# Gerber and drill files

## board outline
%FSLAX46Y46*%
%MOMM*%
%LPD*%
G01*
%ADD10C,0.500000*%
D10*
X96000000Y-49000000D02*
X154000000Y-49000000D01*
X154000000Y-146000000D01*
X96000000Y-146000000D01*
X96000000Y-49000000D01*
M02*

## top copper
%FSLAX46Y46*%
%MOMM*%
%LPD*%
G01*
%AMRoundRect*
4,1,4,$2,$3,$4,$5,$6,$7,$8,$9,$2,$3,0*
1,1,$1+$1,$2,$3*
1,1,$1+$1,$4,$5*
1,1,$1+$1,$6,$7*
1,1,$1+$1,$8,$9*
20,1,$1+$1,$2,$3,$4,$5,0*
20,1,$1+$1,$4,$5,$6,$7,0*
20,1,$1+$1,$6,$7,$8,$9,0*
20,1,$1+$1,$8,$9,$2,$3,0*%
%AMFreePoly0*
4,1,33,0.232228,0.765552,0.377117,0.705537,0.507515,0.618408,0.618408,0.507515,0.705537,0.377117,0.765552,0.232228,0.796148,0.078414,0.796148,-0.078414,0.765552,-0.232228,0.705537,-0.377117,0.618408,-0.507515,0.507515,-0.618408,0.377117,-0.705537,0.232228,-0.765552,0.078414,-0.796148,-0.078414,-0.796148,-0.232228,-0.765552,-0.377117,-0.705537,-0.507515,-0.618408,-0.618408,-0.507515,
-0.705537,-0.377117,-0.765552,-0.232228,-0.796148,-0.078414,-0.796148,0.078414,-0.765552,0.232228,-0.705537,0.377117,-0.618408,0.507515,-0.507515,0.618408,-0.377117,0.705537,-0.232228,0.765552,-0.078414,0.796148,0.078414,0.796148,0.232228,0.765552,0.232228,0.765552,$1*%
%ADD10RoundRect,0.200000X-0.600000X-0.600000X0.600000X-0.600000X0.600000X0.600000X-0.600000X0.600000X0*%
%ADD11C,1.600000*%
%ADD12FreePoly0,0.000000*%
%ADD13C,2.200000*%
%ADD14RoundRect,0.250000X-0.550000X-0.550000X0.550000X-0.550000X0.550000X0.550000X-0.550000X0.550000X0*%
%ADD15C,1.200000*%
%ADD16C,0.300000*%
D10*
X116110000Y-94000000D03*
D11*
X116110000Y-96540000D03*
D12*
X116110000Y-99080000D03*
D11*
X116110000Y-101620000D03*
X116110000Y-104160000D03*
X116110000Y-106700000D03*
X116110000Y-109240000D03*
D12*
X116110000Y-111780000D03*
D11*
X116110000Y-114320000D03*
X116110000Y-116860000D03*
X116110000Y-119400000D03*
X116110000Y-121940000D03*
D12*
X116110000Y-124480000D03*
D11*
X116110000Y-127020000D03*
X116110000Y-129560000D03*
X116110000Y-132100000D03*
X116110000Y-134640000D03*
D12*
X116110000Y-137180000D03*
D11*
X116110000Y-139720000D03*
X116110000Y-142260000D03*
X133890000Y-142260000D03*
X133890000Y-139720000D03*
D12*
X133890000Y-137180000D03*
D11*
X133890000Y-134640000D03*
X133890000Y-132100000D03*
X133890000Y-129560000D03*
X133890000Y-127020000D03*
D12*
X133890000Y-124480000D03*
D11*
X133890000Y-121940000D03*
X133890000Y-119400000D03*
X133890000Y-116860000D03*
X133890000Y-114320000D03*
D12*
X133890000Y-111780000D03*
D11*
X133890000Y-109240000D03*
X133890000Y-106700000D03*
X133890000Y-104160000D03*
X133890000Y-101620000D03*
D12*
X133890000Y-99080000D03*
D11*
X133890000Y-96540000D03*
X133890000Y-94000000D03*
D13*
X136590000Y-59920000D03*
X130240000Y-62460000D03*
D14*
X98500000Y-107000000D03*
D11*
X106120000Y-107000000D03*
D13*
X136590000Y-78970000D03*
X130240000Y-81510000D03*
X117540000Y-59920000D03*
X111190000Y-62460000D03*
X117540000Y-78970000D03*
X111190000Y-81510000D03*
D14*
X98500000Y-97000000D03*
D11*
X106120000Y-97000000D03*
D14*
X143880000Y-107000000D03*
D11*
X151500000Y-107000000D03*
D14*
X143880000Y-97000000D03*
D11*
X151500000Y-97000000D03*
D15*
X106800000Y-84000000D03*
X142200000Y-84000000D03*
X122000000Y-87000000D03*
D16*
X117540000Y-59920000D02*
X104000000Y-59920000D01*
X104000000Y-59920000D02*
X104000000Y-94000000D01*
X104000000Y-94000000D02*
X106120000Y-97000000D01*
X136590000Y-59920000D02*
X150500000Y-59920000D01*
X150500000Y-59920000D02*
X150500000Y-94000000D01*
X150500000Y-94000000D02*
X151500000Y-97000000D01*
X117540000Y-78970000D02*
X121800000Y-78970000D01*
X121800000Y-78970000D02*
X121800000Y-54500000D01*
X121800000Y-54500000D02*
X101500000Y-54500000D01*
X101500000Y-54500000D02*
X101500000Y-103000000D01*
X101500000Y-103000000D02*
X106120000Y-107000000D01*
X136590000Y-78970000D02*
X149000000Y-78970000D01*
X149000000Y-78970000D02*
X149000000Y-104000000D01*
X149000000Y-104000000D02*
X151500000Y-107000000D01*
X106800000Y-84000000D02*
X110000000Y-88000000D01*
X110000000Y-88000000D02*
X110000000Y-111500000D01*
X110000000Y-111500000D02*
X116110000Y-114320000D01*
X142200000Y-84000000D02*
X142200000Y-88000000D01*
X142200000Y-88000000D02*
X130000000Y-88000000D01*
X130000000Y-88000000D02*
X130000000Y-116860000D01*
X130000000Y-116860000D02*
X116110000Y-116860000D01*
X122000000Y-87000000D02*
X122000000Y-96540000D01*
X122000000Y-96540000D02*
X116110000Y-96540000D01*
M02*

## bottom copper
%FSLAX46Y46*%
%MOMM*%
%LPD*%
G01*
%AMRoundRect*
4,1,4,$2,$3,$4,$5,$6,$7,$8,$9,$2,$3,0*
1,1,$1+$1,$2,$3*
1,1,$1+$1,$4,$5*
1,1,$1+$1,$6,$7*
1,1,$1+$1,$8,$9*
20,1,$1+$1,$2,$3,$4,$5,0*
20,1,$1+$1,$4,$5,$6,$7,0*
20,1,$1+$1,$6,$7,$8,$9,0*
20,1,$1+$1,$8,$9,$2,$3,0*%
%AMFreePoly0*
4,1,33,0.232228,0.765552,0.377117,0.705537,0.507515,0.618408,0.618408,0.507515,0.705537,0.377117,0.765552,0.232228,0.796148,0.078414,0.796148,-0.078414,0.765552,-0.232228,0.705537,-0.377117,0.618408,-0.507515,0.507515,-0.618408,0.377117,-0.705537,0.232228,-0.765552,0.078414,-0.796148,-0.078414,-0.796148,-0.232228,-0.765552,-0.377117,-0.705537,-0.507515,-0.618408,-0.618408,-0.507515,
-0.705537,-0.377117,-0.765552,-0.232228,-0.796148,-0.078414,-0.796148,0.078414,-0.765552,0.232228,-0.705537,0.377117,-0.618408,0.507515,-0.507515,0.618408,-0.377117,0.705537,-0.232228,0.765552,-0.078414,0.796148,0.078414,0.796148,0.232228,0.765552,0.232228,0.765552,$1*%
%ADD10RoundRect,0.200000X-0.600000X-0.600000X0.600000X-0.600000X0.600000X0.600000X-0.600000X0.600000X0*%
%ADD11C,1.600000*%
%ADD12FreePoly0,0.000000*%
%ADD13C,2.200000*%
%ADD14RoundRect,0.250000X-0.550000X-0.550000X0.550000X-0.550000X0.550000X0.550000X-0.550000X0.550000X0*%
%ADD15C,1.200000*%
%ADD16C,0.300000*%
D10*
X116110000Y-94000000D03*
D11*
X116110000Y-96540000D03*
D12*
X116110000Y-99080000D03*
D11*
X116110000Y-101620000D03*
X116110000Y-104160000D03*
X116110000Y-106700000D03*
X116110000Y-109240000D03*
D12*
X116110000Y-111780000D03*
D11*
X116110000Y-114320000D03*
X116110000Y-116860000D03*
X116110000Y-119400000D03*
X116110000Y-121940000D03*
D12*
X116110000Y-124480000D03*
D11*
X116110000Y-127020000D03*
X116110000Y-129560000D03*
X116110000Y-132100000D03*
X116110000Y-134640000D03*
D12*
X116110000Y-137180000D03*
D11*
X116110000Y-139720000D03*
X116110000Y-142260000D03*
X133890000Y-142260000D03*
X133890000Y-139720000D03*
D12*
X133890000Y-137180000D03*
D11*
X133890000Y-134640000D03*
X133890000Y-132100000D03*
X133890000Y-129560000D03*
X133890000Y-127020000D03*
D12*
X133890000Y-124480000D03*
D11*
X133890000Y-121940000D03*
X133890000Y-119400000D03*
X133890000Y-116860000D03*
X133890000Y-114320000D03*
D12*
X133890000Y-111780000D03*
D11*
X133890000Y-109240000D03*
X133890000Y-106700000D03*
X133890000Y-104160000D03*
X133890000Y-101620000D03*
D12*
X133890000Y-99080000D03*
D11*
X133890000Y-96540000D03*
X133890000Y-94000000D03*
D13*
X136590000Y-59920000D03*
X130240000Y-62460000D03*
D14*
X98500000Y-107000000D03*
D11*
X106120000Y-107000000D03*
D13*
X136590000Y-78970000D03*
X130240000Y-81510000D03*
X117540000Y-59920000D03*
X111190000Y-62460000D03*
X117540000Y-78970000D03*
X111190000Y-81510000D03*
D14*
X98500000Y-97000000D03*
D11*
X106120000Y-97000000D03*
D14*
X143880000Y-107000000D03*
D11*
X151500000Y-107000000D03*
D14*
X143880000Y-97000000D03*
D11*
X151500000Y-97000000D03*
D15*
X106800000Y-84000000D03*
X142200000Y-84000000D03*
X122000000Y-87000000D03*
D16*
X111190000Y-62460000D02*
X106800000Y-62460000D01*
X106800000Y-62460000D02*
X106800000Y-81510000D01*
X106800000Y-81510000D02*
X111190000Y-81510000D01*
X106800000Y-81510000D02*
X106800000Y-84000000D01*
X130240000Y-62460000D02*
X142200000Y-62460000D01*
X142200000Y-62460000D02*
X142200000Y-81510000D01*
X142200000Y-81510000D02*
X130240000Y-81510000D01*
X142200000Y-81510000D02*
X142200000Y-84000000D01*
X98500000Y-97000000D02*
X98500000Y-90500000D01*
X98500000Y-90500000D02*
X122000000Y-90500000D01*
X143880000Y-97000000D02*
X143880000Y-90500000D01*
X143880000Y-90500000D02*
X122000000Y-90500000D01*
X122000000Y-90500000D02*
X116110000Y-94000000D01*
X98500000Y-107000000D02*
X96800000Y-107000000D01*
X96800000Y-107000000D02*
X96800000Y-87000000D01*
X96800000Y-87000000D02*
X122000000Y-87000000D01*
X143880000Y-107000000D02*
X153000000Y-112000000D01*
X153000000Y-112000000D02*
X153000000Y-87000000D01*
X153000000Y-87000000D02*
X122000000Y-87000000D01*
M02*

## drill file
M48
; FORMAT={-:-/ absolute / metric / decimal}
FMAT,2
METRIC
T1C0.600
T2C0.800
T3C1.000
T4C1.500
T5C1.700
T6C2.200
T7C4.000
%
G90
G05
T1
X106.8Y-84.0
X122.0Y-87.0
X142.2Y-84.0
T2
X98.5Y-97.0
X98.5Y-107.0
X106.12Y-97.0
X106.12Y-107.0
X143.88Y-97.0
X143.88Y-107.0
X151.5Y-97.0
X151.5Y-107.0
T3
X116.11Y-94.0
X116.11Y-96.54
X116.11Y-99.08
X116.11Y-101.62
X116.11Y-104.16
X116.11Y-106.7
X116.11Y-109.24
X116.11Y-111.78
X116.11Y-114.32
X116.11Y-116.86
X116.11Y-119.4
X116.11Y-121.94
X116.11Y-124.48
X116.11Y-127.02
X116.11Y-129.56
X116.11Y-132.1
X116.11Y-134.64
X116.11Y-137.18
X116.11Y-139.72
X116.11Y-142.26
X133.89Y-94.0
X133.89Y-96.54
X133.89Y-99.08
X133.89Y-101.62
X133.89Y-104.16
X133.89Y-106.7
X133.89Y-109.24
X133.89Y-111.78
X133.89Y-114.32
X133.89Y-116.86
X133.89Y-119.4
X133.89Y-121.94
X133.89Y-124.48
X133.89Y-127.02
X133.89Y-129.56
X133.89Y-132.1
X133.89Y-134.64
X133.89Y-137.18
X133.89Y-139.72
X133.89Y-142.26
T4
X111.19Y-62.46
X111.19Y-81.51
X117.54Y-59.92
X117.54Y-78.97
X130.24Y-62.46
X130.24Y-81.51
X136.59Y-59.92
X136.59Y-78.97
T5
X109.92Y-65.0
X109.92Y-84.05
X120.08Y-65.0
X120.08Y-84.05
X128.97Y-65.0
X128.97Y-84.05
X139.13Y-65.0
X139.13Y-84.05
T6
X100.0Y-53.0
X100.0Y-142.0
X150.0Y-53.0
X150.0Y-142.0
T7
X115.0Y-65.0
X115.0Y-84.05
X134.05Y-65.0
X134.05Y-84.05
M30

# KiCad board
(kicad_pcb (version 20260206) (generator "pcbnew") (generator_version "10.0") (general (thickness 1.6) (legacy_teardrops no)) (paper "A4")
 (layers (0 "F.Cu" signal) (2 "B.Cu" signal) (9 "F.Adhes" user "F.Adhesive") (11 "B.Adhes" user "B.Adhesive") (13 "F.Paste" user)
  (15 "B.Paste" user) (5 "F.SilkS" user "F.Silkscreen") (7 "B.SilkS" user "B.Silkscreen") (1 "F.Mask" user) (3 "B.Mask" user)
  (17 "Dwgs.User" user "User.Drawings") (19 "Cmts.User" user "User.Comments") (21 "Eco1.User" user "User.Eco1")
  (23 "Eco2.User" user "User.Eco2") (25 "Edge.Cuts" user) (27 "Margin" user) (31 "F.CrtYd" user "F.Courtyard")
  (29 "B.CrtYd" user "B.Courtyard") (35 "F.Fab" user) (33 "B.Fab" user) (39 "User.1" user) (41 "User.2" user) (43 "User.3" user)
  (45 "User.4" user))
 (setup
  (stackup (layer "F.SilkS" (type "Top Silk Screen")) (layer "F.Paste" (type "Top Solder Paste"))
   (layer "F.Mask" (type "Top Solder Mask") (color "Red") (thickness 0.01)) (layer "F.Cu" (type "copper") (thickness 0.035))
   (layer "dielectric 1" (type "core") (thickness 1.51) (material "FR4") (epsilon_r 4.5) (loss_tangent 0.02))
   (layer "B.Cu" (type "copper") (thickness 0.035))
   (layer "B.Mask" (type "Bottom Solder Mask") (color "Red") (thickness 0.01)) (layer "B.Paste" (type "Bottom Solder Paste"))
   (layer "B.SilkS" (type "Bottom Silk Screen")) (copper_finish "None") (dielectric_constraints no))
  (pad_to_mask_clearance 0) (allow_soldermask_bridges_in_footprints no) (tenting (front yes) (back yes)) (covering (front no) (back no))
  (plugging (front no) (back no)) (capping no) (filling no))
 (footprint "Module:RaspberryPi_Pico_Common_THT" (layer "F.Cu") (at 116.11 94)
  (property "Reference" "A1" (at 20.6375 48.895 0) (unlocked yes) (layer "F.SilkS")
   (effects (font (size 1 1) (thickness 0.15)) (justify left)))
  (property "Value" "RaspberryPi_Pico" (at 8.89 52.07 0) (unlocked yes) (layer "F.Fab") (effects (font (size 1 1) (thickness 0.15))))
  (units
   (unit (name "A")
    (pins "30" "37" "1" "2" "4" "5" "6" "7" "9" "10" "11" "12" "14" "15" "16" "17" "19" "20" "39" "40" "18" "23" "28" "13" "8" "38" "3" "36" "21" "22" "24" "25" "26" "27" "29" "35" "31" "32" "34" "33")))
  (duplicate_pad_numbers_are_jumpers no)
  (pad "1" thru_hole roundrect (at 0 0) (size 1.6 1.6) (drill 1) (layers "*.Cu" "*.Mask") (remove_unused_layers no) (roundrect_rratio 0.125)
   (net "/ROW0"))
  (pad "2" thru_hole circle (at 0 2.54) (size 1.6 1.6) (drill 1) (layers "*.Cu" "*.Mask") (remove_unused_layers no) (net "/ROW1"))
  (pad "3" thru_hole custom (at 0 5.08) (size 1.6 1.6) (drill 1) (layers "*.Cu" "*.Mask") (remove_unused_layers no)
   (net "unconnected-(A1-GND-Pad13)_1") (options (clearance outline) (anchor circle)) (primitives))
  (pad "4" thru_hole circle (at 0 7.62) (size 1.6 1.6) (drill 1) (layers "*.Cu" "*.Mask") (remove_unused_layers no)
   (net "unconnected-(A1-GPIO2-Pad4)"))
  (pad "5" thru_hole circle (at 0 10.16) (size 1.6 1.6) (drill 1) (layers "*.Cu" "*.Mask") (remove_unused_layers no)
   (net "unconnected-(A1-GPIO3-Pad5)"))
  (pad "6" thru_hole circle (at 0 12.7) (size 1.6 1.6) (drill 1) (layers "*.Cu" "*.Mask") (remove_unused_layers no)
   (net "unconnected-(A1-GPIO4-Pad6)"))
  (pad "7" thru_hole circle (at 0 15.24) (size 1.6 1.6) (drill 1) (layers "*.Cu" "*.Mask") (remove_unused_layers no)
   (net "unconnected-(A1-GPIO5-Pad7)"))
  (pad "8" thru_hole custom (at 0 17.78) (size 1.6 1.6) (drill 1) (layers "*.Cu" "*.Mask") (remove_unused_layers no)
   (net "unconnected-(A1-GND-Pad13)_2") (options (clearance outline) (anchor circle)) (primitives))
  (pad "9" thru_hole circle (at 0 20.32) (size 1.6 1.6) (drill 1) (layers "*.Cu" "*.Mask") (remove_unused_layers no) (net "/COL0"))
  (pad "10" thru_hole circle (at 0 22.86) (size 1.6 1.6) (drill 1) (layers "*.Cu" "*.Mask") (remove_unused_layers no) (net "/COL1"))
  (pad "11" thru_hole circle (at 0 25.4) (size 1.6 1.6) (drill 1) (layers "*.Cu" "*.Mask") (remove_unused_layers no)
   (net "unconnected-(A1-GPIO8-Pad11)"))
  (pad "12" thru_hole circle (at 0 27.94) (size 1.6 1.6) (drill 1) (layers "*.Cu" "*.Mask") (remove_unused_layers no)
   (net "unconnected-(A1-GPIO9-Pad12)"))
  (pad "13" thru_hole custom (at 0 30.48) (size 1.6 1.6) (drill 1) (layers "*.Cu" "*.Mask") (remove_unused_layers no)
   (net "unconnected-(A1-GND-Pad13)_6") (options (clearance outline) (anchor circle)) (primitives))
  (pad "14" thru_hole circle (at 0 33.02) (size 1.6 1.6) (drill 1) (layers "*.Cu" "*.Mask") (remove_unused_layers no)
   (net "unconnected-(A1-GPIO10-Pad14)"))
  (pad "15" thru_hole circle (at 0 35.56) (size 1.6 1.6) (drill 1) (layers "*.Cu" "*.Mask") (remove_unused_layers no)
   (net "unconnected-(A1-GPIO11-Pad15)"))
  (pad "16" thru_hole circle (at 0 38.1) (size 1.6 1.6) (drill 1) (layers "*.Cu" "*.Mask") (remove_unused_layers no)
   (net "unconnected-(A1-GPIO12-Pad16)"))
  (pad "17" thru_hole circle (at 0 40.64) (size 1.6 1.6) (drill 1) (layers "*.Cu" "*.Mask") (remove_unused_layers no)
   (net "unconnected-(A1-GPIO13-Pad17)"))
  (pad "18" thru_hole custom (at 0 43.18) (size 1.6 1.6) (drill 1) (layers "*.Cu" "*.Mask") (remove_unused_layers no)
   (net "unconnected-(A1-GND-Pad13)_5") (options (clearance outline) (anchor circle)) (primitives))
  (pad "19" thru_hole circle (at 0 45.72) (size 1.6 1.6) (drill 1) (layers "*.Cu" "*.Mask") (remove_unused_layers no)
   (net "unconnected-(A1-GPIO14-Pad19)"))
  (pad "20" thru_hole circle (at 0 48.26) (size 1.6 1.6) (drill 1) (layers "*.Cu" "*.Mask") (remove_unused_layers no)
   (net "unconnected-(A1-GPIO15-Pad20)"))
  (pad "21" thru_hole circle (at 17.78 48.26) (size 1.6 1.6) (drill 1) (layers "*.Cu" "*.Mask") (remove_unused_layers no)
   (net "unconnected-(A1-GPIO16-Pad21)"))
  (pad "22" thru_hole circle (at 17.78 45.72) (size 1.6 1.6) (drill 1) (layers "*.Cu" "*.Mask") (remove_unused_layers no)
   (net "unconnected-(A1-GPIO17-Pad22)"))
  (pad "23" thru_hole custom (at 17.78 43.18) (size 1.6 1.6) (drill 1) (layers "*.Cu" "*.Mask") (remove_unused_layers no)
   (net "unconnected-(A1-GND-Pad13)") (options (clearance outline) (anchor circle)) (primitives))
  (pad "24" thru_hole circle (at 17.78 40.64) (size 1.6 1.6) (drill 1) (layers "*.Cu" "*.Mask") (remove_unused_layers no)
   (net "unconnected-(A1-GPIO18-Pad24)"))
  (pad "25" thru_hole circle (at 17.78 38.1) (size 1.6 1.6) (drill 1) (layers "*.Cu" "*.Mask") (remove_unused_layers no)
   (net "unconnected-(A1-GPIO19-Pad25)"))
  (pad "26" thru_hole circle (at 17.78 35.56) (size 1.6 1.6) (drill 1) (layers "*.Cu" "*.Mask") (remove_unused_layers no)
   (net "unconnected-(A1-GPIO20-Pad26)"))
  (pad "27" thru_hole circle (at 17.78 33.02) (size 1.6 1.6) (drill 1) (layers "*.Cu" "*.Mask") (remove_unused_layers no)
   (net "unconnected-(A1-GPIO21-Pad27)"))
  (pad "28" thru_hole custom (at 17.78 30.48) (size 1.6 1.6) (drill 1) (layers "*.Cu" "*.Mask") (remove_unused_layers no)
   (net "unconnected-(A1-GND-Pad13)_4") (options (clearance outline) (anchor circle)) (primitives))
  (pad "29" thru_hole circle (at 17.78 27.94) (size 1.6 1.6) (drill 1) (layers "*.Cu" "*.Mask") (remove_unused_layers no)
   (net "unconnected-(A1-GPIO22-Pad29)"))
  (pad "30" thru_hole circle (at 17.78 25.4) (size 1.6 1.6) (drill 1) (layers "*.Cu" "*.Mask") (remove_unused_layers no)
   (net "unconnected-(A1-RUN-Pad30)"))
  (pad "31" thru_hole circle (at 17.78 22.86) (size 1.6 1.6) (drill 1) (layers "*.Cu" "*.Mask") (remove_unused_layers no)
   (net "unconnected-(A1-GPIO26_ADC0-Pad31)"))
  (pad "32" thru_hole circle (at 17.78 20.32) (size 1.6 1.6) (drill 1) (layers "*.Cu" "*.Mask") (remove_unused_layers no)
   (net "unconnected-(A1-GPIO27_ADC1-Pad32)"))
  (pad "33" thru_hole custom (at 17.78 17.78) (size 1.6 1.6) (drill 1) (layers "*.Cu" "*.Mask") (remove_unused_layers no)
   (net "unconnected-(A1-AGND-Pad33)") (options (clearance outline) (anchor circle)) (primitives))
  (pad "34" thru_hole circle (at 17.78 15.24) (size 1.6 1.6) (drill 1) (layers "*.Cu" "*.Mask") (remove_unused_layers no)
   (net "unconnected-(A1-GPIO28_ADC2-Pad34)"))
  (pad "35" thru_hole circle (at 17.78 12.7) (size 1.6 1.6) (drill 1) (layers "*.Cu" "*.Mask") (remove_unused_layers no)
   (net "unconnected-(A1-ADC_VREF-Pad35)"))
  (pad "36" thru_hole circle (at 17.78 10.16) (size 1.6 1.6) (drill 1) (layers "*.Cu" "*.Mask") (remove_unused_layers no)
   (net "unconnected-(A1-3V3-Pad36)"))
  (pad "37" thru_hole circle (at 17.78 7.62) (size 1.6 1.6) (drill 1) (layers "*.Cu" "*.Mask") (remove_unused_layers no)
   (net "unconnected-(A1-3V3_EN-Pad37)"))
  (pad "38" thru_hole custom (at 17.78 5.08) (size 1.6 1.6) (drill 1) (layers "*.Cu" "*.Mask") (remove_unused_layers no)
   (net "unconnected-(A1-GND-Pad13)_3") (options (clearance outline) (anchor circle)) (primitives))
  (pad "39" thru_hole circle (at 17.78 2.54) (size 1.6 1.6) (drill 1) (layers "*.Cu" "*.Mask") (remove_unused_layers no)
   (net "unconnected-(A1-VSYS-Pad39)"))
  (pad "40" thru_hole circle (at 17.78 0) (size 1.6 1.6) (drill 1) (layers "*.Cu" "*.Mask") (remove_unused_layers no)
   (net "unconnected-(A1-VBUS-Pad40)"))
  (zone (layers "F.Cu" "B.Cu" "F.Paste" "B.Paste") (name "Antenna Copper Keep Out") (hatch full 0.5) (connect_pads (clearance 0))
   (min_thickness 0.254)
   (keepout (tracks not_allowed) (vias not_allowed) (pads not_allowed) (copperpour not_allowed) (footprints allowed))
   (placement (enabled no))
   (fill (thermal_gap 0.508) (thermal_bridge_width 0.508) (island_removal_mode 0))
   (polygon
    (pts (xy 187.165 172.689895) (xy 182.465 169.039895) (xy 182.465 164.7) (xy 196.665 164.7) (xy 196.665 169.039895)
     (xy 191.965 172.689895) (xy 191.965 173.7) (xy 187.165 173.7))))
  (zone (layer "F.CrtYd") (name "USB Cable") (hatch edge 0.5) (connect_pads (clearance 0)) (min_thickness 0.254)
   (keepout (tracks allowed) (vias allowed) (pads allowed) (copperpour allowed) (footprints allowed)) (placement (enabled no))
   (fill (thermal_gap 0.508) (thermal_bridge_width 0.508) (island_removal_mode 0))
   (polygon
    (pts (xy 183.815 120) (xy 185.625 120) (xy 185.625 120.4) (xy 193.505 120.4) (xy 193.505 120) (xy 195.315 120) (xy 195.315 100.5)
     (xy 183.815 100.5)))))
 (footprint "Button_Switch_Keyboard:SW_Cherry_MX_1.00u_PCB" (layer "F.Cu") (at 136.59 59.92)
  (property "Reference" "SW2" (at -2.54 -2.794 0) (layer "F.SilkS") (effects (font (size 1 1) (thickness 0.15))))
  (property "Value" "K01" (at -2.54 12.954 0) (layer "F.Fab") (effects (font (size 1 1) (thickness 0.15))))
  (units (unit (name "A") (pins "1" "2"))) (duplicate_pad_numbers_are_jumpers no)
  (pad "" np_thru_hole circle (at -7.62 5.08) (size 1.7 1.7) (drill 1.7) (layers "*.Cu" "*.Mask"))
  (pad "" np_thru_hole circle (at -2.54 5.08) (size 4 4) (drill 4) (layers "*.Cu" "*.Mask"))
  (pad "" np_thru_hole circle (at 2.54 5.08) (size 1.7 1.7) (drill 1.7) (layers "*.Cu" "*.Mask"))
  (pad "1" thru_hole circle (at 0 0) (size 2.2 2.2) (drill 1.5) (layers "*.Cu" "*.Mask") (remove_unused_layers no) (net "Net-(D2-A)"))
  (pad "2" thru_hole circle (at -6.35 2.54) (size 2.2 2.2) (drill 1.5) (layers "*.Cu" "*.Mask") (remove_unused_layers no) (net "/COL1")))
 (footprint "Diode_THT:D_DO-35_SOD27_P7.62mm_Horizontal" (layer "F.Cu") (at 98.5 107)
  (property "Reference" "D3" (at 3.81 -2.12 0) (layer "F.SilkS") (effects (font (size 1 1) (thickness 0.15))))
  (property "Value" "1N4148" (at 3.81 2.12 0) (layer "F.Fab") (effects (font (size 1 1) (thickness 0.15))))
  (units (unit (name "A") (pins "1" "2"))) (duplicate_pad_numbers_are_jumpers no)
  (pad "1" thru_hole roundrect (at 0 0) (size 1.6 1.6) (drill 0.8) (layers "*.Cu" "*.Mask") (remove_unused_layers no)
   (roundrect_rratio 0.15625) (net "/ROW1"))
  (pad "2" thru_hole circle (at 7.62 0) (size 1.6 1.6) (drill 0.8) (layers "*.Cu" "*.Mask") (remove_unused_layers no) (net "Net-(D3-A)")))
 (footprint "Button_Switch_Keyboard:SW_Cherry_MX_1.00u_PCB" (layer "F.Cu") (at 136.59 78.97)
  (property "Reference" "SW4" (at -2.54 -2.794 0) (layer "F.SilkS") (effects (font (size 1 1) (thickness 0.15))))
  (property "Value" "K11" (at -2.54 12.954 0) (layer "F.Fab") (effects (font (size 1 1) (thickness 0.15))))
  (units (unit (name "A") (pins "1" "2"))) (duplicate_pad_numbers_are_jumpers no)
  (pad "" np_thru_hole circle (at -7.62 5.08) (size 1.7 1.7) (drill 1.7) (layers "*.Cu" "*.Mask"))
  (pad "" np_thru_hole circle (at -2.54 5.08) (size 4 4) (drill 4) (layers "*.Cu" "*.Mask"))
  (pad "" np_thru_hole circle (at 2.54 5.08) (size 1.7 1.7) (drill 1.7) (layers "*.Cu" "*.Mask"))
  (pad "1" thru_hole circle (at 0 0) (size 2.2 2.2) (drill 1.5) (layers "*.Cu" "*.Mask") (remove_unused_layers no) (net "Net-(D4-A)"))
  (pad "2" thru_hole circle (at -6.35 2.54) (size 2.2 2.2) (drill 1.5) (layers "*.Cu" "*.Mask") (remove_unused_layers no) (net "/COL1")))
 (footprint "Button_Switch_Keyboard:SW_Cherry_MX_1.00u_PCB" (layer "F.Cu") (at 117.54 59.92)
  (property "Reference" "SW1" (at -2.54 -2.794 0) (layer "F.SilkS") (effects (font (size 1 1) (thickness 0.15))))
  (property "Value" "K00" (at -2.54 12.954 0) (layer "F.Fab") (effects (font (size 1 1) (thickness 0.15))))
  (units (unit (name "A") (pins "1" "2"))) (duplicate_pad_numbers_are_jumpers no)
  (pad "" np_thru_hole circle (at -7.62 5.08) (size 1.7 1.7) (drill 1.7) (layers "*.Cu" "*.Mask"))
  (pad "" np_thru_hole circle (at -2.54 5.08) (size 4 4) (drill 4) (layers "*.Cu" "*.Mask"))
  (pad "" np_thru_hole circle (at 2.54 5.08) (size 1.7 1.7) (drill 1.7) (layers "*.Cu" "*.Mask"))
  (pad "1" thru_hole circle (at 0 0) (size 2.2 2.2) (drill 1.5) (layers "*.Cu" "*.Mask") (remove_unused_layers no) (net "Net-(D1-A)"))
  (pad "2" thru_hole circle (at -6.35 2.54) (size 2.2 2.2) (drill 1.5) (layers "*.Cu" "*.Mask") (remove_unused_layers no) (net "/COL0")))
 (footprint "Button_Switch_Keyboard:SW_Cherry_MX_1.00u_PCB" (layer "F.Cu") (at 117.54 78.97)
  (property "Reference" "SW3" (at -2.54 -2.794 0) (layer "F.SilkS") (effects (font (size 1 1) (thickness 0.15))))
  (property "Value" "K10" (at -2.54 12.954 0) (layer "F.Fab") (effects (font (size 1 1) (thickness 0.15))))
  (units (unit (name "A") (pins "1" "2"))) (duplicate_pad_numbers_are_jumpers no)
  (pad "" np_thru_hole circle (at -7.62 5.08) (size 1.7 1.7) (drill 1.7) (layers "*.Cu" "*.Mask"))
  (pad "" np_thru_hole circle (at -2.54 5.08) (size 4 4) (drill 4) (layers "*.Cu" "*.Mask"))
  (pad "" np_thru_hole circle (at 2.54 5.08) (size 1.7 1.7) (drill 1.7) (layers "*.Cu" "*.Mask"))
  (pad "1" thru_hole circle (at 0 0) (size 2.2 2.2) (drill 1.5) (layers "*.Cu" "*.Mask") (remove_unused_layers no) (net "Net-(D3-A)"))
  (pad "2" thru_hole circle (at -6.35 2.54) (size 2.2 2.2) (drill 1.5) (layers "*.Cu" "*.Mask") (remove_unused_layers no) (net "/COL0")))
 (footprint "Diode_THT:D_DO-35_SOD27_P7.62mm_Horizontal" (layer "F.Cu") (at 98.5 97)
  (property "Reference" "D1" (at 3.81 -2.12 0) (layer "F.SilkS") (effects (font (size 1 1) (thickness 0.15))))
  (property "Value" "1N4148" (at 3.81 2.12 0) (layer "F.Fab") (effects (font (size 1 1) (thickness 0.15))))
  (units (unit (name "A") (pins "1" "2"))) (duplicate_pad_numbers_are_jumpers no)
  (pad "1" thru_hole roundrect (at 0 0) (size 1.6 1.6) (drill 0.8) (layers "*.Cu" "*.Mask") (remove_unused_layers no)
   (roundrect_rratio 0.15625) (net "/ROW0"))
  (pad "2" thru_hole circle (at 7.62 0) (size 1.6 1.6) (drill 0.8) (layers "*.Cu" "*.Mask") (remove_unused_layers no) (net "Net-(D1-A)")))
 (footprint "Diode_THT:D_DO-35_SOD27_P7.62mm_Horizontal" (layer "F.Cu") (at 143.88 107)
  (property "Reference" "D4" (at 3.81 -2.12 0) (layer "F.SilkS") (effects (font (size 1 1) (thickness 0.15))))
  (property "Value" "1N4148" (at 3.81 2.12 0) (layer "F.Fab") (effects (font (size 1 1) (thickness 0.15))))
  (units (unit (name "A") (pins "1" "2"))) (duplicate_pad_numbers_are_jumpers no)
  (pad "1" thru_hole roundrect (at 0 0) (size 1.6 1.6) (drill 0.8) (layers "*.Cu" "*.Mask") (remove_unused_layers no)
   (roundrect_rratio 0.15625) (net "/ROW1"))
  (pad "2" thru_hole circle (at 7.62 0) (size 1.6 1.6) (drill 0.8) (layers "*.Cu" "*.Mask") (remove_unused_layers no) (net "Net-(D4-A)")))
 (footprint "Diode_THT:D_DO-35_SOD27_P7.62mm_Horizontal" (layer "F.Cu") (at 143.88 97)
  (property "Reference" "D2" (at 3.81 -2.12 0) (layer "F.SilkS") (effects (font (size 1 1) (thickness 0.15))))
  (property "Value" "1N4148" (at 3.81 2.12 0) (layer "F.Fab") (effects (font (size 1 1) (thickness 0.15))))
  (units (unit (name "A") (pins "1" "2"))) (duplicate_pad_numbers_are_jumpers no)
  (pad "1" thru_hole roundrect (at 0 0) (size 1.6 1.6) (drill 0.8) (layers "*.Cu" "*.Mask") (remove_unused_layers no)
   (roundrect_rratio 0.15625) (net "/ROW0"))
  (pad "2" thru_hole circle (at 7.62 0) (size 1.6 1.6) (drill 0.8) (layers "*.Cu" "*.Mask") (remove_unused_layers no) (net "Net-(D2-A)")))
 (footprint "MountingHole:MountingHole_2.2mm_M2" (layer "F.Cu") (at 100 53)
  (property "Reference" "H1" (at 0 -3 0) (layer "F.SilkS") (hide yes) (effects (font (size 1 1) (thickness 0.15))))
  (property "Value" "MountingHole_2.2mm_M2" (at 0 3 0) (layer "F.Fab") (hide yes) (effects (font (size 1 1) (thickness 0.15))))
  (pad "" np_thru_hole circle (at 0 0) (size 2.2 2.2) (drill 2.2) (layers "*.Cu" "*.Mask")))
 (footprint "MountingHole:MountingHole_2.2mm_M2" (layer "F.Cu") (at 150 53)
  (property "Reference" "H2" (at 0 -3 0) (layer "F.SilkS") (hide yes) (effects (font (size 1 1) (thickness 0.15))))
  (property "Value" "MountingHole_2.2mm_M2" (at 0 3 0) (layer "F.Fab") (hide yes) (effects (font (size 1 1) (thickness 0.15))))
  (pad "" np_thru_hole circle (at 0 0) (size 2.2 2.2) (drill 2.2) (layers "*.Cu" "*.Mask")))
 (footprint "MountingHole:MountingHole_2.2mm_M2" (layer "F.Cu") (at 100 142)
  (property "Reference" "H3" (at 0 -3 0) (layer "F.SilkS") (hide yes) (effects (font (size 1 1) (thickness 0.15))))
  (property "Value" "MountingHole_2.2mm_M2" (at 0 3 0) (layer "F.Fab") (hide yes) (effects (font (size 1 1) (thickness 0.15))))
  (pad "" np_thru_hole circle (at 0 0) (size 2.2 2.2) (drill 2.2) (layers "*.Cu" "*.Mask")))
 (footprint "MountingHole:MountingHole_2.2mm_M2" (layer "F.Cu") (at 150 142)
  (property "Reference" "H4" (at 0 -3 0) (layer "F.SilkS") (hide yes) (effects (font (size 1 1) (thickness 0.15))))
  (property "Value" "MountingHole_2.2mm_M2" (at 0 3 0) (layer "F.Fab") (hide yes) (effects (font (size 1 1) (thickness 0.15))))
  (pad "" np_thru_hole circle (at 0 0) (size 2.2 2.2) (drill 2.2) (layers "*.Cu" "*.Mask")))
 (gr_rect (start 96 49) (end 154 146) (stroke (width 0.5) (type solid)) (fill none) (layer "Edge.Cuts"))
 (segment (start 117.54 59.92) (end 104 59.92) (width 0.3) (layer "F.Cu") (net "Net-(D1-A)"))
 (segment (start 104 59.92) (end 104 94) (width 0.3) (layer "F.Cu") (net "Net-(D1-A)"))
 (segment (start 104 94) (end 106.12 97) (width 0.3) (layer "F.Cu") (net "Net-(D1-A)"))
 (segment (start 136.59 59.92) (end 150.5 59.92) (width 0.3) (layer "F.Cu") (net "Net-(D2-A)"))
 (segment (start 150.5 59.92) (end 150.5 94) (width 0.3) (layer "F.Cu") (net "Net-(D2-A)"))
 (segment (start 150.5 94) (end 151.5 97) (width 0.3) (layer "F.Cu") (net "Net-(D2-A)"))
 (segment (start 117.54 78.97) (end 121.8 78.97) (width 0.3) (layer "F.Cu") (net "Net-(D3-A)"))
 (segment (start 121.8 78.97) (end 121.8 54.5) (width 0.3) (layer "F.Cu") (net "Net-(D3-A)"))
 (segment (start 121.8 54.5) (end 101.5 54.5) (width 0.3) (layer "F.Cu") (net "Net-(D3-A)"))
 (segment (start 101.5 54.5) (end 101.5 103) (width 0.3) (layer "F.Cu") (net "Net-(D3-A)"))
 (segment (start 101.5 103) (end 106.12 107) (width 0.3) (layer "F.Cu") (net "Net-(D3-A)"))
 (segment (start 136.59 78.97) (end 149 78.97) (width 0.3) (layer "F.Cu") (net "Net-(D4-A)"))
 (segment (start 149 78.97) (end 149 104) (width 0.3) (layer "F.Cu") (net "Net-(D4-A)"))
 (segment (start 149 104) (end 151.5 107) (width 0.3) (layer "F.Cu") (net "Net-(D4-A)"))
 (segment (start 111.19 62.46) (end 106.8 62.46) (width 0.3) (layer "B.Cu") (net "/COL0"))
 (segment (start 106.8 62.46) (end 106.8 81.51) (width 0.3) (layer "B.Cu") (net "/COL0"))
 (segment (start 106.8 81.51) (end 111.19 81.51) (width 0.3) (layer "B.Cu") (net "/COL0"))
 (segment (start 106.8 81.51) (end 106.8 84) (width 0.3) (layer "B.Cu") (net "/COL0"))
 (segment (start 130.24 62.46) (end 142.2 62.46) (width 0.3) (layer "B.Cu") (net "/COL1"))
 (segment (start 142.2 62.46) (end 142.2 81.51) (width 0.3) (layer "B.Cu") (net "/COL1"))
 (segment (start 142.2 81.51) (end 130.24 81.51) (width 0.3) (layer "B.Cu") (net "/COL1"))
 (segment (start 142.2 81.51) (end 142.2 84) (width 0.3) (layer "B.Cu") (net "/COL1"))
 (segment (start 106.8 84) (end 110 88) (width 0.3) (layer "F.Cu") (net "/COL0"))
 (segment (start 110 88) (end 110 111.5) (width 0.3) (layer "F.Cu") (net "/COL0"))
 (segment (start 110 111.5) (end 116.11 114.32) (width 0.3) (layer "F.Cu") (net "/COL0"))
 (segment (start 142.2 84) (end 142.2 88) (width 0.3) (layer "F.Cu") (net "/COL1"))
 (segment (start 142.2 88) (end 130 88) (width 0.3) (layer "F.Cu") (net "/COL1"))
 (segment (start 130 88) (end 130 116.86) (width 0.3) (layer "F.Cu") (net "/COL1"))
 (segment (start 130 116.86) (end 116.11 116.86) (width 0.3) (layer "F.Cu") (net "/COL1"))
 (segment (start 98.5 97) (end 98.5 90.5) (width 0.3) (layer "B.Cu") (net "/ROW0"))
 (segment (start 98.5 90.5) (end 122 90.5) (width 0.3) (layer "B.Cu") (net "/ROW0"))
 (segment (start 143.88 97) (end 143.88 90.5) (width 0.3) (layer "B.Cu") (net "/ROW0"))
 (segment (start 143.88 90.5) (end 122 90.5) (width 0.3) (layer "B.Cu") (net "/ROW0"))
 (segment (start 122 90.5) (end 116.11 94) (width 0.3) (layer "B.Cu") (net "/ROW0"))
 (segment (start 98.5 107) (end 96.8 107) (width 0.3) (layer "B.Cu") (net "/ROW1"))
 (segment (start 96.8 107) (end 96.8 87) (width 0.3) (layer "B.Cu") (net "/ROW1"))
 (segment (start 96.8 87) (end 122 87) (width 0.3) (layer "B.Cu") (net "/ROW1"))
 (segment (start 143.88 107) (end 153 112) (width 0.3) (layer "B.Cu") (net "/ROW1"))
 (segment (start 153 112) (end 153 87) (width 0.3) (layer "B.Cu") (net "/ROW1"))
 (segment (start 153 87) (end 122 87) (width 0.3) (layer "B.Cu") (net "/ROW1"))
 (segment (start 122 87) (end 122 96.54) (width 0.3) (layer "F.Cu") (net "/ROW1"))
 (segment (start 122 96.54) (end 116.11 96.54) (width 0.3) (layer "F.Cu") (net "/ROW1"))
 (via (at 106.8 84) (size 1.2) (drill 0.6) (layers "F.Cu" "B.Cu") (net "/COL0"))
 (via (at 142.2 84) (size 1.2) (drill 0.6) (layers "F.Cu" "B.Cu") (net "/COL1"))
 (via (at 122 87) (size 1.2) (drill 0.6) (layers "F.Cu" "B.Cu") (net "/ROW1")))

